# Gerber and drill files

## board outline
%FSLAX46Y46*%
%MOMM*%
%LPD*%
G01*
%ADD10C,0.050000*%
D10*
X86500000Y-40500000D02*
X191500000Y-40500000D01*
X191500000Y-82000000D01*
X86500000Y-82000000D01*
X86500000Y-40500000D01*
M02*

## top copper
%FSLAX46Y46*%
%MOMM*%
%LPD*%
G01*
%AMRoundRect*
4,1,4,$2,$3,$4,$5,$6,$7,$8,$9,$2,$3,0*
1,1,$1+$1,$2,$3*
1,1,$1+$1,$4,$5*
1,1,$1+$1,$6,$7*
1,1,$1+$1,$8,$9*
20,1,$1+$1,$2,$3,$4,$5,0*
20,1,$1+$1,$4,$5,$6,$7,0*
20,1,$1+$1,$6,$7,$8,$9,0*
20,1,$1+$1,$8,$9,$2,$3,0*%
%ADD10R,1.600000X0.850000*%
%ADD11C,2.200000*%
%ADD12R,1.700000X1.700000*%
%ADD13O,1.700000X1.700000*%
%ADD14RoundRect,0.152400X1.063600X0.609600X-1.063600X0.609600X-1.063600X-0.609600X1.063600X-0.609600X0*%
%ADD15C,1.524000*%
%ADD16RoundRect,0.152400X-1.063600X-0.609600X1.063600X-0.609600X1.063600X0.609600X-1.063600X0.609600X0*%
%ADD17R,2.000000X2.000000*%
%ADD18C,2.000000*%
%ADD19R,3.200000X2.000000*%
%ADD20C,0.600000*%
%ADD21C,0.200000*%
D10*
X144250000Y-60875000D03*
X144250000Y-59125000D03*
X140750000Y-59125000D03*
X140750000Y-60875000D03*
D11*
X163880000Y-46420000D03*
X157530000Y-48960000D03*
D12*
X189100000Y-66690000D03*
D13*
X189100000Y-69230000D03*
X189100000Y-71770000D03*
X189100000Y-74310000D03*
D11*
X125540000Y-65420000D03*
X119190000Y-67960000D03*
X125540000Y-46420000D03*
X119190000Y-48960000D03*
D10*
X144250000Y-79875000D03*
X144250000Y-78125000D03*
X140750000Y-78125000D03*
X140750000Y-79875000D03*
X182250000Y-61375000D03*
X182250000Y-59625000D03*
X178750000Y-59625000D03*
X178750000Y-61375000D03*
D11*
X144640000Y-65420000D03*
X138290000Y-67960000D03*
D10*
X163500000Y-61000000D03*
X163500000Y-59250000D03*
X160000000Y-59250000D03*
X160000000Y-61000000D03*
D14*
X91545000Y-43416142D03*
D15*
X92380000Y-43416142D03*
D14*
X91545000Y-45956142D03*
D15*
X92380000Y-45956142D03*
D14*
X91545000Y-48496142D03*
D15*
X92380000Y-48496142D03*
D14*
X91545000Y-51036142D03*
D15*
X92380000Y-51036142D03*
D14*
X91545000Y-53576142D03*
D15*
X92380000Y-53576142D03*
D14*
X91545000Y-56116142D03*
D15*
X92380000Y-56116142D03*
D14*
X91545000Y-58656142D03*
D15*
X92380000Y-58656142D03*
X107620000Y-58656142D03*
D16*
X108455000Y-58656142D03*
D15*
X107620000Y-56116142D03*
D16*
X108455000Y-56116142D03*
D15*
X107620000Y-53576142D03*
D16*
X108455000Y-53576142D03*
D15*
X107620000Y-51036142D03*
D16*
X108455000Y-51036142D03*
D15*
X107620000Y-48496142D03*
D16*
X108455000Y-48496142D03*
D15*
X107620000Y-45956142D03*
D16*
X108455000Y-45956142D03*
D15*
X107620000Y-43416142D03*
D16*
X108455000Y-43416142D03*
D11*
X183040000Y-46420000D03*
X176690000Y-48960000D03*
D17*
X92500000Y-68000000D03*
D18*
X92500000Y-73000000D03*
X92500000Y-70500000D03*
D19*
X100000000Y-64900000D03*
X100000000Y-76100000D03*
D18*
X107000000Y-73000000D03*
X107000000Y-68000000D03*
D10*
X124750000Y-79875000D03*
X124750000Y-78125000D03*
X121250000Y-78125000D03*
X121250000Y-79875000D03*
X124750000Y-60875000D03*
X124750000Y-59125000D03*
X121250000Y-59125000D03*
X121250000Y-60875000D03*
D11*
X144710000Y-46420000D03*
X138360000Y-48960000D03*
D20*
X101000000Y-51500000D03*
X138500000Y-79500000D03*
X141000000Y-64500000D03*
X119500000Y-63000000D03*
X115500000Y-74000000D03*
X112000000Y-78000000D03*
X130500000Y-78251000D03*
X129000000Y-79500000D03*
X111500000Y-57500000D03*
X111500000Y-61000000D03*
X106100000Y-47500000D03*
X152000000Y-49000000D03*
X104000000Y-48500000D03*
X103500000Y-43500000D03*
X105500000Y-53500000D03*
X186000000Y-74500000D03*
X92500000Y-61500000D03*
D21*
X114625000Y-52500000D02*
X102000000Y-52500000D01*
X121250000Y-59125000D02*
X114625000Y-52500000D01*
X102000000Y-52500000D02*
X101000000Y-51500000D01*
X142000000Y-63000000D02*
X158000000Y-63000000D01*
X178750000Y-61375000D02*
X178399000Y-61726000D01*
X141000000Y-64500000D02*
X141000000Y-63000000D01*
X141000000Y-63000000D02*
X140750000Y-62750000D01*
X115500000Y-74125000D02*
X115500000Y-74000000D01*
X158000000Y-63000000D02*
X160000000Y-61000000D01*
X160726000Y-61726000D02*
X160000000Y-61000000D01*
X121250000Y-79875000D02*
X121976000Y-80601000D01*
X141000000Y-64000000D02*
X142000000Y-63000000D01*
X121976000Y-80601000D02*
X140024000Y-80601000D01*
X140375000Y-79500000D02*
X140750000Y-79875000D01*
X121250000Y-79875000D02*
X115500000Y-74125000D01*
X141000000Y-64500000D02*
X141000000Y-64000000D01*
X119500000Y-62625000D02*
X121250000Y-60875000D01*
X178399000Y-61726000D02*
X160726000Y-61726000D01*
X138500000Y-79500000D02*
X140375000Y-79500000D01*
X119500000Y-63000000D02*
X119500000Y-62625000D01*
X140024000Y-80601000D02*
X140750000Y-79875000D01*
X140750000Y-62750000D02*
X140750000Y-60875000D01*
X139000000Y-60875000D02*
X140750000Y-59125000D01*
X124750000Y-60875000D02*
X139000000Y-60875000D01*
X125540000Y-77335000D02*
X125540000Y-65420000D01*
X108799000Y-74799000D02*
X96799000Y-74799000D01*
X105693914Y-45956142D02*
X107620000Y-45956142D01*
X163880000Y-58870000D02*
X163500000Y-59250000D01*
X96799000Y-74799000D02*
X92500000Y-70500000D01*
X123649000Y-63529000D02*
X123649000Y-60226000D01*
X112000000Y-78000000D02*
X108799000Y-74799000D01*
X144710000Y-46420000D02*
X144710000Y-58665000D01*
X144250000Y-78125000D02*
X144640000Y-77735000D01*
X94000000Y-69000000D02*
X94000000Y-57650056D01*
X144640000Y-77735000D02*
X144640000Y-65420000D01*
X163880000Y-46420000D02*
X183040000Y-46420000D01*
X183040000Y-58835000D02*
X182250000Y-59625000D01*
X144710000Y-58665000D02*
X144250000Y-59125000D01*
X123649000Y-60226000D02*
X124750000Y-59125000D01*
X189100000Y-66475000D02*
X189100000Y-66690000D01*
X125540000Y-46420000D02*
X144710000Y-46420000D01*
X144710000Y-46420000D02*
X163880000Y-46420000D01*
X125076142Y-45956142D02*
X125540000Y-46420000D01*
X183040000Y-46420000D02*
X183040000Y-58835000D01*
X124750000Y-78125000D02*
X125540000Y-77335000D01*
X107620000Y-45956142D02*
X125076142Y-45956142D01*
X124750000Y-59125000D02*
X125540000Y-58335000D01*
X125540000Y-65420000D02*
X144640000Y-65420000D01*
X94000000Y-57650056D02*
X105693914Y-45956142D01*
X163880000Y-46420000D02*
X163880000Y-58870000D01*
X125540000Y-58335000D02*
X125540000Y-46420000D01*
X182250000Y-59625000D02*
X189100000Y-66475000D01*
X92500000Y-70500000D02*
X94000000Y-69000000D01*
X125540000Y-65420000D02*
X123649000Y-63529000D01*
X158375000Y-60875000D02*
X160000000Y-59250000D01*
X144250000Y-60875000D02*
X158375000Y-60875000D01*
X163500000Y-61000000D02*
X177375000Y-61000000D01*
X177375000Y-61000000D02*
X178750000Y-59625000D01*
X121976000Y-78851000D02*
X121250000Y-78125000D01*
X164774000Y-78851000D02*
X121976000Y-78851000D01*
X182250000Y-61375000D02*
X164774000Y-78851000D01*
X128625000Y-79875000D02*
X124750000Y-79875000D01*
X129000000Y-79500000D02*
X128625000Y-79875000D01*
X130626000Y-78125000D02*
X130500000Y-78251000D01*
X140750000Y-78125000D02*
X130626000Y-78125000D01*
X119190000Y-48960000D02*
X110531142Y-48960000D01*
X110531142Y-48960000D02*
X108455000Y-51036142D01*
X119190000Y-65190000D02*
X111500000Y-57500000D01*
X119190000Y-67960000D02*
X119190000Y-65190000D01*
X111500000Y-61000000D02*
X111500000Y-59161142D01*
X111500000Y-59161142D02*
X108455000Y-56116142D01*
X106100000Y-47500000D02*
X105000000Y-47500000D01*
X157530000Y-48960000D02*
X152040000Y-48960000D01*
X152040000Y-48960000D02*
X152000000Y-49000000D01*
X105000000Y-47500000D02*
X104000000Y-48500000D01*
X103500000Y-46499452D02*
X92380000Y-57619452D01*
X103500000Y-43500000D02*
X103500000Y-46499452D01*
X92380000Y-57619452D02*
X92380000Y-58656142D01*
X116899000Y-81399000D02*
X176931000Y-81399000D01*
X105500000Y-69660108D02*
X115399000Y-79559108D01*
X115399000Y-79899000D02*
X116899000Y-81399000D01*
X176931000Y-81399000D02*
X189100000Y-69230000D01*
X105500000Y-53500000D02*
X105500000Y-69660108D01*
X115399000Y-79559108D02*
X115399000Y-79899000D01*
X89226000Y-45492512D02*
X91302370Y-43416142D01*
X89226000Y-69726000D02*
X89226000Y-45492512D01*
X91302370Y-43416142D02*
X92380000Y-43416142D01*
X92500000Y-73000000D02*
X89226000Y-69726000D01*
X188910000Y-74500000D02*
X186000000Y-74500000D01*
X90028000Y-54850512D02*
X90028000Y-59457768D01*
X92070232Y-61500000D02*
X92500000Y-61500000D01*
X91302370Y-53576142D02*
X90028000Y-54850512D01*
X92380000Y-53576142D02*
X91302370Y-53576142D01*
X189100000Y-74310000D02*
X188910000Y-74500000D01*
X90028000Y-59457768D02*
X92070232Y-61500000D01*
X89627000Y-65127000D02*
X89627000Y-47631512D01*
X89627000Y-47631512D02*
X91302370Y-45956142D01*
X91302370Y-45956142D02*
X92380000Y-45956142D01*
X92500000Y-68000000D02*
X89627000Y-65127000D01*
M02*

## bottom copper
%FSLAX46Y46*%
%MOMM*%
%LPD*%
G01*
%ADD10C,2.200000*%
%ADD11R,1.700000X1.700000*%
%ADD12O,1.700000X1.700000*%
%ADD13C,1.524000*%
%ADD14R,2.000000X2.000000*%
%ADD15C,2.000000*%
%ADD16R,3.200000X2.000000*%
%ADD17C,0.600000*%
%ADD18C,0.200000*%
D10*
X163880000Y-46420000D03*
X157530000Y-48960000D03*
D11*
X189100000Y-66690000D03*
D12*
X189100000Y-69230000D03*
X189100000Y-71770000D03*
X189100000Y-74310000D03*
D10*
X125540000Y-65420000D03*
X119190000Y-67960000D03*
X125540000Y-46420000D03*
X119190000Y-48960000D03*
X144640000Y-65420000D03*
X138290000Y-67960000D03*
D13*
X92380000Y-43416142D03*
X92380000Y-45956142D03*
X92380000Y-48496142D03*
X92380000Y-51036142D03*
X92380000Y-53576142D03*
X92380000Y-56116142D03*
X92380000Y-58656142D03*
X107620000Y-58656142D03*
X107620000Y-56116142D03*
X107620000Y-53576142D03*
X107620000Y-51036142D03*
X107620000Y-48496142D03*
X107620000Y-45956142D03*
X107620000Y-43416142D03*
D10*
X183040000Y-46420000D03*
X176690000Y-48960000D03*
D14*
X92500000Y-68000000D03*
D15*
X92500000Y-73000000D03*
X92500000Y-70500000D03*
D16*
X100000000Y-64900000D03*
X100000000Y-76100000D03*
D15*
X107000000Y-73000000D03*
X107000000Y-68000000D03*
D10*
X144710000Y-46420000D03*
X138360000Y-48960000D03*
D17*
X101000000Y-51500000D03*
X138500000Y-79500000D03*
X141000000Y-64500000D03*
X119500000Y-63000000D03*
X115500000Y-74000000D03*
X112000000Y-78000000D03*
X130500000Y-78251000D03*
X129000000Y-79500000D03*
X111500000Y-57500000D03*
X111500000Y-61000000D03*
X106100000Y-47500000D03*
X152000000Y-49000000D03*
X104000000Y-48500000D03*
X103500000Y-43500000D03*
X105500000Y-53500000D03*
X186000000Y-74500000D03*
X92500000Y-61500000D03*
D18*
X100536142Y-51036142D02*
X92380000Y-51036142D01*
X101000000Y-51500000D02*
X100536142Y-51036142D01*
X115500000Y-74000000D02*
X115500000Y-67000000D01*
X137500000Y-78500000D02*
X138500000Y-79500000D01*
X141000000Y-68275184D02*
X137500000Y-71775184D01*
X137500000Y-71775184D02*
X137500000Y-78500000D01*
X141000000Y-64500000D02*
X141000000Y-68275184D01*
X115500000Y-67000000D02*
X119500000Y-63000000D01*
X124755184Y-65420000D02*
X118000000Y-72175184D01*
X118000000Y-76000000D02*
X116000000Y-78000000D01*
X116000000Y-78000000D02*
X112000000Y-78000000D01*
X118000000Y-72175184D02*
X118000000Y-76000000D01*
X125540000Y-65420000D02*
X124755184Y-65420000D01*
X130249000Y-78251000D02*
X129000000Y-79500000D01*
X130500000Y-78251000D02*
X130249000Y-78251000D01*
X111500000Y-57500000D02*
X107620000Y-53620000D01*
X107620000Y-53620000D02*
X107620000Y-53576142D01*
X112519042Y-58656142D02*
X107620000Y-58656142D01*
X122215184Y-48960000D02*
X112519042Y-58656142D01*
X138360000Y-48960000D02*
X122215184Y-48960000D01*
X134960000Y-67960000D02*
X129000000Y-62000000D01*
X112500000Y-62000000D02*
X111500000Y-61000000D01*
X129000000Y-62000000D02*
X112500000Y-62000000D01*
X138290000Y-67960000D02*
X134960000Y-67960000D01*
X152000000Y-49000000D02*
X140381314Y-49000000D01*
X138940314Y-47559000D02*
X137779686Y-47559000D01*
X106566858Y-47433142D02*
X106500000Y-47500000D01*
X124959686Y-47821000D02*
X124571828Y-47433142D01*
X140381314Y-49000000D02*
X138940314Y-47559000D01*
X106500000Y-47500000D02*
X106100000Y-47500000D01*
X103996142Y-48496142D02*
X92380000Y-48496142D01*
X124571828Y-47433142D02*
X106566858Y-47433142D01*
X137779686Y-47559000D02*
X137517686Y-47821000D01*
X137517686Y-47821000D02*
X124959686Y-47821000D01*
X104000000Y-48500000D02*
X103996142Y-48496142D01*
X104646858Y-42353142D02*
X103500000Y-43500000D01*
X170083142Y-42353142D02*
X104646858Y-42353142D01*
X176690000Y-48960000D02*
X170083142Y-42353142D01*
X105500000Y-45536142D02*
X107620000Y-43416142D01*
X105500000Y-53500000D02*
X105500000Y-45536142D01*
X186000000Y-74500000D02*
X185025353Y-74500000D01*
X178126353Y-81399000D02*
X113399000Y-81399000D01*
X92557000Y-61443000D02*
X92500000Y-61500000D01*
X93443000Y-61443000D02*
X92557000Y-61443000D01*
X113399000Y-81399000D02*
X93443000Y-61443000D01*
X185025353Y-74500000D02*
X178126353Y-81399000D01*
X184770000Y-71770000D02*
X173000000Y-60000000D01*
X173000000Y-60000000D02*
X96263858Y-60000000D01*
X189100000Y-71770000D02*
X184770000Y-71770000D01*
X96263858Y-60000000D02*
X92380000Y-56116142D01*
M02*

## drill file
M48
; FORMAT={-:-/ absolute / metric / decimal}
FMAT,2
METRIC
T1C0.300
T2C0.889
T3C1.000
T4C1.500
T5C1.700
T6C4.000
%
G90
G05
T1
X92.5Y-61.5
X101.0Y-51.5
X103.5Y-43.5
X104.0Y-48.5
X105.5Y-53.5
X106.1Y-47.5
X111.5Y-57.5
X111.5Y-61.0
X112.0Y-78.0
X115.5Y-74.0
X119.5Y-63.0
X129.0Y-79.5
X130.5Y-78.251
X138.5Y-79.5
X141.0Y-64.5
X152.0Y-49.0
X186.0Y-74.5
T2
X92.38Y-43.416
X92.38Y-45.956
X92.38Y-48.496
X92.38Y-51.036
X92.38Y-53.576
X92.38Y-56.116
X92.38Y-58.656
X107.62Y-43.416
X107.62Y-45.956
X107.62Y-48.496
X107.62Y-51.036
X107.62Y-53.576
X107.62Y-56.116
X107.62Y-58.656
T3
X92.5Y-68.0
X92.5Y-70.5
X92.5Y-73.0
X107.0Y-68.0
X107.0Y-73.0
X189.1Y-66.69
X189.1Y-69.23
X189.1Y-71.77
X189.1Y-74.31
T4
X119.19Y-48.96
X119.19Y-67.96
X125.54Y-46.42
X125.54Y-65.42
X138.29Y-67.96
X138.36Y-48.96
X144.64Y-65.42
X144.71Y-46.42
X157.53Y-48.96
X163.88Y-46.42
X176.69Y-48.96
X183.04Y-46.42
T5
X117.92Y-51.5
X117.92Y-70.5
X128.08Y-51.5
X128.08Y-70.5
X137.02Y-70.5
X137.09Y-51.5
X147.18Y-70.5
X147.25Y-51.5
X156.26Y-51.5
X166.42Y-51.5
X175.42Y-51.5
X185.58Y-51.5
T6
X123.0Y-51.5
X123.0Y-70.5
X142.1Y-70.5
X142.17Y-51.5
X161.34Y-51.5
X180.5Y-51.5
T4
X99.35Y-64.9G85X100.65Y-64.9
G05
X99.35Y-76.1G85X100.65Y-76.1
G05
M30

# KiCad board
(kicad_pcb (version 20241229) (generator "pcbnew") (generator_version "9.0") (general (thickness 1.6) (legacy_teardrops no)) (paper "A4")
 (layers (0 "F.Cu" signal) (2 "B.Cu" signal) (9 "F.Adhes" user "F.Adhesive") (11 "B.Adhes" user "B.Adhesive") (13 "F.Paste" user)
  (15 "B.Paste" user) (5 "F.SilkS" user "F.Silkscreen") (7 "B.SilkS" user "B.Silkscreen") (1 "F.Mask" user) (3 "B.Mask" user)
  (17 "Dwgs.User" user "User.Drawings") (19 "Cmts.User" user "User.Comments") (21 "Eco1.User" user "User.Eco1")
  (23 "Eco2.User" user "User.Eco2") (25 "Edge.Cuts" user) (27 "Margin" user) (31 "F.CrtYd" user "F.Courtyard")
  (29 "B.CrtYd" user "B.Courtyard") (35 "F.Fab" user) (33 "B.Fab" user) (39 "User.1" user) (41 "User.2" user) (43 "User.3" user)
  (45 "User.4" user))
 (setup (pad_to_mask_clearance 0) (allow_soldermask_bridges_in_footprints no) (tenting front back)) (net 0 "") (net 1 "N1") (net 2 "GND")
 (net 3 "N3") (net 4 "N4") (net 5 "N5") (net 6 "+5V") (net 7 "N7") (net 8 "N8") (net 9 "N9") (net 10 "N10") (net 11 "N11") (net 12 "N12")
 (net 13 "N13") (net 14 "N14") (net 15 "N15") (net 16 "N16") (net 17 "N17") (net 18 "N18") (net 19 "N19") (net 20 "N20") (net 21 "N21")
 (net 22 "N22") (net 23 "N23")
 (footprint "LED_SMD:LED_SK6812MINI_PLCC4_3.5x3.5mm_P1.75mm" (layer "F.Cu") (at 142.5 60 180)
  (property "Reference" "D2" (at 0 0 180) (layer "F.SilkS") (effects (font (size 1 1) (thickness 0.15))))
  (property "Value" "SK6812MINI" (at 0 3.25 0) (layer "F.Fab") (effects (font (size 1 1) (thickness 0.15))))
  (pad "1" smd rect (at -1.75 -0.875 180) (size 1.6 0.85) (layers "F.Cu" "F.Mask" "F.Paste") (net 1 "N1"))
  (pad "2" smd rect (at -1.75 0.875 180) (size 1.6 0.85) (layers "F.Cu" "F.Mask" "F.Paste") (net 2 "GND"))
  (pad "3" smd rect (at 1.75 0.875 180) (size 1.6 0.85) (layers "F.Cu" "F.Mask" "F.Paste") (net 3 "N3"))
  (pad "4" smd rect (at 1.75 -0.875 180) (size 1.6 0.85) (layers "F.Cu" "F.Mask" "F.Paste") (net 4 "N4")))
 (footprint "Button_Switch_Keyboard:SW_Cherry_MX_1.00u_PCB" (layer "F.Cu") (at 163.88 46.42)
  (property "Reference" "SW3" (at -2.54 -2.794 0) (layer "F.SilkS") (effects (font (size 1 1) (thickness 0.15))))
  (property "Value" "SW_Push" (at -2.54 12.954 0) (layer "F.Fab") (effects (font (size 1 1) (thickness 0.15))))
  (pad "" np_thru_hole circle (at -7.62 5.08) (size 1.7 1.7) (drill 1.7) (layers "*.Cu" "*.Mask"))
  (pad "" np_thru_hole circle (at -2.54 5.08) (size 4 4) (drill 4) (layers "*.Cu" "*.Mask"))
  (pad "" np_thru_hole circle (at 2.54 5.08) (size 1.7 1.7) (drill 1.7) (layers "*.Cu" "*.Mask"))
  (pad "1" thru_hole circle (at 0 0) (size 2.2 2.2) (drill 1.5) (layers "*.Cu" "*.Mask") (remove_unused_layers no) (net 2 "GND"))
  (pad "2" thru_hole circle (at -6.35 2.54) (size 2.2 2.2) (drill 1.5) (layers "*.Cu" "*.Mask") (remove_unused_layers no) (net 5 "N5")))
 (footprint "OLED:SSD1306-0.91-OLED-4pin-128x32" (layer "F.Cu") (at 152.6 64.5)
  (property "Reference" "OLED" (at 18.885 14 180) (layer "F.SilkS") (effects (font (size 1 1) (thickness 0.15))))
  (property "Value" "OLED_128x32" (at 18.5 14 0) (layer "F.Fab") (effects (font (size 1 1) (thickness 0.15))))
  (pad "1" thru_hole rect (at 36.5 2.19) (size 1.7 1.7) (drill 1) (layers "*.Cu" "*.Mask") (remove_unused_layers no) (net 2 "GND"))
  (pad "2" thru_hole oval (at 36.5 4.73) (size 1.7 1.7) (drill 1) (layers "*.Cu" "*.Mask") (remove_unused_layers no) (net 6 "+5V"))
  (pad "3" thru_hole oval (at 36.5 7.27) (size 1.7 1.7) (drill 1) (layers "*.Cu" "*.Mask") (remove_unused_layers no) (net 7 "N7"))
  (pad "4" thru_hole oval (at 36.5 9.81) (size 1.7 1.7) (drill 1) (layers "*.Cu" "*.Mask") (remove_unused_layers no) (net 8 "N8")))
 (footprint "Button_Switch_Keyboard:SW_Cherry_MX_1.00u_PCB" (layer "F.Cu") (at 125.54 65.42)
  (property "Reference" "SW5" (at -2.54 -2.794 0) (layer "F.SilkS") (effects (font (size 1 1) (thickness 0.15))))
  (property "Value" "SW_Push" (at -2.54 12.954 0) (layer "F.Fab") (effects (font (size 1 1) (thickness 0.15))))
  (pad "" np_thru_hole circle (at -7.62 5.08) (size 1.7 1.7) (drill 1.7) (layers "*.Cu" "*.Mask"))
  (pad "" np_thru_hole circle (at -2.54 5.08) (size 4 4) (drill 4) (layers "*.Cu" "*.Mask"))
  (pad "" np_thru_hole circle (at 2.54 5.08) (size 1.7 1.7) (drill 1.7) (layers "*.Cu" "*.Mask"))
  (pad "1" thru_hole circle (at 0 0) (size 2.2 2.2) (drill 1.5) (layers "*.Cu" "*.Mask") (remove_unused_layers no) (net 2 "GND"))
  (pad "2" thru_hole circle (at -6.35 2.54) (size 2.2 2.2) (drill 1.5) (layers "*.Cu" "*.Mask") (remove_unused_layers no) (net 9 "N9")))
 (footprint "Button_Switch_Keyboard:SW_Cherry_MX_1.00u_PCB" (layer "F.Cu") (at 125.54 46.42)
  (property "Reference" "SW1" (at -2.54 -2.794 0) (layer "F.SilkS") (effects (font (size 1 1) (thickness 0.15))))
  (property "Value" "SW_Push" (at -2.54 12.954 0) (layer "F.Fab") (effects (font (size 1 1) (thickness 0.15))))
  (pad "" np_thru_hole circle (at -7.62 5.08) (size 1.7 1.7) (drill 1.7) (layers "*.Cu" "*.Mask"))
  (pad "" np_thru_hole circle (at -2.54 5.08) (size 4 4) (drill 4) (layers "*.Cu" "*.Mask"))
  (pad "" np_thru_hole circle (at 2.54 5.08) (size 1.7 1.7) (drill 1.7) (layers "*.Cu" "*.Mask"))
  (pad "1" thru_hole circle (at 0 0) (size 2.2 2.2) (drill 1.5) (layers "*.Cu" "*.Mask") (remove_unused_layers no) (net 2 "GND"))
  (pad "2" thru_hole circle (at -6.35 2.54) (size 2.2 2.2) (drill 1.5) (layers "*.Cu" "*.Mask") (remove_unused_layers no) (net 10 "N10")))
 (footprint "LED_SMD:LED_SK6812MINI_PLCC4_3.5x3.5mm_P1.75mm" (layer "F.Cu") (at 142.5 79 180)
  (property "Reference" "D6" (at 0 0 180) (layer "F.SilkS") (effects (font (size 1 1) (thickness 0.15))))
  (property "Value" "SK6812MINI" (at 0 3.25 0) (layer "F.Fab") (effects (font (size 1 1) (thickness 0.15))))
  (pad "1" smd rect (at -1.75 -0.875 180) (size 1.6 0.85) (layers "F.Cu" "F.Mask" "F.Paste") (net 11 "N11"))
  (pad "2" smd rect (at -1.75 0.875 180) (size 1.6 0.85) (layers "F.Cu" "F.Mask" "F.Paste") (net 2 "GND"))
  (pad "3" smd rect (at 1.75 0.875 180) (size 1.6 0.85) (layers "F.Cu" "F.Mask" "F.Paste") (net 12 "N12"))
  (pad "4" smd rect (at 1.75 -0.875 180) (size 1.6 0.85) (layers "F.Cu" "F.Mask" "F.Paste") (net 4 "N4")))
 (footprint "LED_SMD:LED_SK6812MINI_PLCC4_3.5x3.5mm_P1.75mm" (layer "F.Cu") (at 180.5 60.5 180)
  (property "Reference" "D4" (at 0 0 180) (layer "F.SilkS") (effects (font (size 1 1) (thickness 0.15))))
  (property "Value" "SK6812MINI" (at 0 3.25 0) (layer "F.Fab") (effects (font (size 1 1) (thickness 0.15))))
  (pad "1" smd rect (at -1.75 -0.875 180) (size 1.6 0.85) (layers "F.Cu" "F.Mask" "F.Paste") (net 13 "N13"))
  (pad "2" smd rect (at -1.75 0.875 180) (size 1.6 0.85) (layers "F.Cu" "F.Mask" "F.Paste") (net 2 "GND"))
  (pad "3" smd rect (at 1.75 0.875 180) (size 1.6 0.85) (layers "F.Cu" "F.Mask" "F.Paste") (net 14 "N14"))
  (pad "4" smd rect (at 1.75 -0.875 180) (size 1.6 0.85) (layers "F.Cu" "F.Mask" "F.Paste") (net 4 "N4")))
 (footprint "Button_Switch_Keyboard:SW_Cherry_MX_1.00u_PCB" (layer "F.Cu") (at 144.64 65.42)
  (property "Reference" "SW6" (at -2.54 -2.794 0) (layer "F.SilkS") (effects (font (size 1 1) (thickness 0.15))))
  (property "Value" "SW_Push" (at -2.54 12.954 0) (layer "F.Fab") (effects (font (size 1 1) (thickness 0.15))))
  (pad "" np_thru_hole circle (at -7.62 5.08) (size 1.7 1.7) (drill 1.7) (layers "*.Cu" "*.Mask"))
  (pad "" np_thru_hole circle (at -2.54 5.08) (size 4 4) (drill 4) (layers "*.Cu" "*.Mask"))
  (pad "" np_thru_hole circle (at 2.54 5.08) (size 1.7 1.7) (drill 1.7) (layers "*.Cu" "*.Mask"))
  (pad "1" thru_hole circle (at 0 0) (size 2.2 2.2) (drill 1.5) (layers "*.Cu" "*.Mask") (remove_unused_layers no) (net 2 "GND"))
  (pad "2" thru_hole circle (at -6.35 2.54) (size 2.2 2.2) (drill 1.5) (layers "*.Cu" "*.Mask") (remove_unused_layers no) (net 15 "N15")))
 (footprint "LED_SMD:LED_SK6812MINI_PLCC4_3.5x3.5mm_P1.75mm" (layer "F.Cu") (at 161.75 60.125 180)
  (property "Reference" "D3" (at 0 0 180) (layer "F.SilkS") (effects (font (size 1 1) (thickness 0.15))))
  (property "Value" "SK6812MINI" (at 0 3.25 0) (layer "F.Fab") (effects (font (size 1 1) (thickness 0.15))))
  (pad "1" smd rect (at -1.75 -0.875 180) (size 1.6 0.85) (layers "F.Cu" "F.Mask" "F.Paste") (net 14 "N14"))
  (pad "2" smd rect (at -1.75 0.875 180) (size 1.6 0.85) (layers "F.Cu" "F.Mask" "F.Paste") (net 2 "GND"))
  (pad "3" smd rect (at 1.75 0.875 180) (size 1.6 0.85) (layers "F.Cu" "F.Mask" "F.Paste") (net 1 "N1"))
  (pad "4" smd rect (at 1.75 -0.875 180) (size 1.6 0.85) (layers "F.Cu" "F.Mask" "F.Paste") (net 4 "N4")))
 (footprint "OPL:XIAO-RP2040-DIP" (layer "F.Cu") (at 100 51.036142)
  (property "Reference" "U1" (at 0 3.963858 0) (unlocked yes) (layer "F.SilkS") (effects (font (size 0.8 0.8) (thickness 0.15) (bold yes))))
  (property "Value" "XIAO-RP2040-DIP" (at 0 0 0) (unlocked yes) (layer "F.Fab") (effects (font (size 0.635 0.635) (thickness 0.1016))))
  (pad "1" smd roundrect (at -8.455 -7.62 180) (size 2.432 1.524) (layers "F.Cu" "F.Mask") (roundrect_rratio 0.1) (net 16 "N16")
   (thermal_bridge_angle 45))
  (pad "1" thru_hole circle (at -7.62 -7.62 180) (size 1.524 1.524) (drill 0.889) (layers "*.Cu" "*.Mask") (remove_unused_layers no)
   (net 16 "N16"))
  (pad "2" smd roundrect (at -8.455 -5.08 180) (size 2.432 1.524) (layers "F.Cu" "F.Mask") (roundrect_rratio 0.1) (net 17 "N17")
   (thermal_bridge_angle 45))
  (pad "2" thru_hole circle (at -7.62 -5.08 180) (size 1.524 1.524) (drill 0.889) (layers "*.Cu" "*.Mask") (remove_unused_layers no)
   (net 17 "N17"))
  (pad "3" smd roundrect (at -8.455 -2.54 180) (size 2.432 1.524) (layers "F.Cu" "F.Mask") (roundrect_rratio 0.1) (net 5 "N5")
   (thermal_bridge_angle 45))
  (pad "3" thru_hole circle (at -7.62 -2.54 180) (size 1.524 1.524) (drill 0.889) (layers "*.Cu" "*.Mask") (remove_unused_layers no)
   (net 5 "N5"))
  (pad "4" smd roundrect (at -8.455 0 180) (size 2.432 1.524) (layers "F.Cu" "F.Mask") (roundrect_rratio 0.1) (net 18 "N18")
   (thermal_bridge_angle 45))
  (pad "4" thru_hole circle (at -7.62 0 180) (size 1.524 1.524) (drill 0.889) (layers "*.Cu" "*.Mask") (remove_unused_layers no)
   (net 18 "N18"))
  (pad "5" smd roundrect (at -8.455 2.54 180) (size 2.432 1.524) (layers "F.Cu" "F.Mask") (roundrect_rratio 0.1) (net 8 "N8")
   (thermal_bridge_angle 45))
  (pad "5" thru_hole circle (at -7.62 2.54 180) (size 1.524 1.524) (drill 0.889) (layers "*.Cu" "*.Mask") (remove_unused_layers no)
   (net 8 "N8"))
  (pad "6" smd roundrect (at -8.455 5.08 180) (size 2.432 1.524) (layers "F.Cu" "F.Mask") (roundrect_rratio 0.1) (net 7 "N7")
   (thermal_bridge_angle 45))
  (pad "6" thru_hole circle (at -7.62 5.08 180) (size 1.524 1.524) (drill 0.889) (layers "*.Cu" "*.Mask") (remove_unused_layers no)
   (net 7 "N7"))
  (pad "7" smd roundrect (at -8.455 7.62 180) (size 2.432 1.524) (layers "F.Cu" "F.Mask") (roundrect_rratio 0.1) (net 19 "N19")
   (thermal_bridge_angle 45))
  (pad "7" thru_hole circle (at -7.62 7.62 180) (size 1.524 1.524) (drill 0.889) (layers "*.Cu" "*.Mask") (remove_unused_layers no)
   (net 19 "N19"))
  (pad "8" thru_hole circle (at 7.62 7.62) (size 1.524 1.524) (drill 0.889) (layers "*.Cu" "*.Mask") (remove_unused_layers no)
   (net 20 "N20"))
  (pad "8" smd roundrect (at 8.455 7.62) (size 2.432 1.524) (layers "F.Cu" "F.Mask") (roundrect_rratio 0.1) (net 20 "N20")
   (thermal_bridge_angle 45))
  (pad "9" thru_hole circle (at 7.62 5.08) (size 1.524 1.524) (drill 0.889) (layers "*.Cu" "*.Mask") (remove_unused_layers no)
   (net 15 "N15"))
  (pad "9" smd roundrect (at 8.455 5.08) (size 2.432 1.524) (layers "F.Cu" "F.Mask") (roundrect_rratio 0.1) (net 15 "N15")
   (thermal_bridge_angle 45))
  (pad "10" thru_hole circle (at 7.62 2.54) (size 1.524 1.524) (drill 0.889) (layers "*.Cu" "*.Mask") (remove_unused_layers no) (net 9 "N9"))
  (pad "10" smd roundrect (at 8.455 2.54) (size 2.432 1.524) (layers "F.Cu" "F.Mask") (roundrect_rratio 0.1) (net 9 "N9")
   (thermal_bridge_angle 45))
  (pad "11" thru_hole circle (at 7.62 0) (size 1.524 1.524) (drill 0.889) (layers "*.Cu" "*.Mask") (remove_unused_layers no) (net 10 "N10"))
  (pad "11" smd roundrect (at 8.455 0) (size 2.432 1.524) (layers "F.Cu" "F.Mask") (roundrect_rratio 0.1) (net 10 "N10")
   (thermal_bridge_angle 45))
  (pad "12" thru_hole circle (at 7.62 -2.54) (size 1.524 1.524) (drill 0.889) (layers "*.Cu" "*.Mask") (remove_unused_layers no)
   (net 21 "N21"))
  (pad "12" smd roundrect (at 8.455 -2.54) (size 2.432 1.524) (layers "F.Cu" "F.Mask") (roundrect_rratio 0.1) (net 21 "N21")
   (thermal_bridge_angle 45))
  (pad "13" thru_hole circle (at 7.62 -5.08) (size 1.524 1.524) (drill 0.889) (layers "*.Cu" "*.Mask") (remove_unused_layers no)
   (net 2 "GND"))
  (pad "13" smd roundrect (at 8.455 -5.08) (size 2.432 1.524) (layers "F.Cu" "F.Mask") (roundrect_rratio 0.1) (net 2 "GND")
   (thermal_bridge_angle 45))
  (pad "14" thru_hole circle (at 7.62 -7.62) (size 1.524 1.524) (drill 0.889) (layers "*.Cu" "*.Mask") (remove_unused_layers no)
   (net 6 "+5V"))
  (pad "14" smd roundrect (at 8.455 -7.62) (size 2.432 1.524) (layers "F.Cu" "F.Mask") (roundrect_rratio 0.1) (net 6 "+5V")
   (thermal_bridge_angle 45)))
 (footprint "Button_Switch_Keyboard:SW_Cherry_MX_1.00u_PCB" (layer "F.Cu") (at 183.04 46.42)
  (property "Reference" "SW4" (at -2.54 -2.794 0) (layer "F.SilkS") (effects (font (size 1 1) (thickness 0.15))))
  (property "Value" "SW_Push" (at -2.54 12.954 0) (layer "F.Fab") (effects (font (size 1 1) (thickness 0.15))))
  (pad "" np_thru_hole circle (at -7.62 5.08) (size 1.7 1.7) (drill 1.7) (layers "*.Cu" "*.Mask"))
  (pad "" np_thru_hole circle (at -2.54 5.08) (size 4 4) (drill 4) (layers "*.Cu" "*.Mask"))
  (pad "" np_thru_hole circle (at 2.54 5.08) (size 1.7 1.7) (drill 1.7) (layers "*.Cu" "*.Mask"))
  (pad "1" thru_hole circle (at 0 0) (size 2.2 2.2) (drill 1.5) (layers "*.Cu" "*.Mask") (remove_unused_layers no) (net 2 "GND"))
  (pad "2" thru_hole circle (at -6.35 2.54) (size 2.2 2.2) (drill 1.5) (layers "*.Cu" "*.Mask") (remove_unused_layers no) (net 19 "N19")))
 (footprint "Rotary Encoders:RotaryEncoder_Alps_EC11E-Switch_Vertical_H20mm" (layer "F.Cu") (at 92.5 68)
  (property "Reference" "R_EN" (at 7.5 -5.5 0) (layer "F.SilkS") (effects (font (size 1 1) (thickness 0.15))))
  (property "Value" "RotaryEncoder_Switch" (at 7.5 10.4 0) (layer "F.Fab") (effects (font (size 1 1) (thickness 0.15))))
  (pad "A" thru_hole rect (at 0 0) (size 2 2) (drill 1) (layers "*.Cu" "*.Mask") (remove_unused_layers no) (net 17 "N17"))
  (pad "B" thru_hole circle (at 0 5) (size 2 2) (drill 1) (layers "*.Cu" "*.Mask") (remove_unused_layers no) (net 16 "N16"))
  (pad "C" thru_hole circle (at 0 2.5) (size 2 2) (drill 1) (layers "*.Cu" "*.Mask") (remove_unused_layers no) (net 2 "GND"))
  (pad "MP" thru_hole rect (at 7.5 -3.1) (size 3.2 2) (drill oval 2.8 1.5) (layers "*.Cu" "*.Mask") (remove_unused_layers no))
  (pad "MP" thru_hole rect (at 7.5 8.1) (size 3.2 2) (drill oval 2.8 1.5) (layers "*.Cu" "*.Mask") (remove_unused_layers no))
  (pad "S1" thru_hole circle (at 14.5 5) (size 2 2) (drill 1) (layers "*.Cu" "*.Mask") (remove_unused_layers no) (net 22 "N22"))
  (pad "S2" thru_hole circle (at 14.5 0) (size 2 2) (drill 1) (layers "*.Cu" "*.Mask") (remove_unused_layers no) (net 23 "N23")))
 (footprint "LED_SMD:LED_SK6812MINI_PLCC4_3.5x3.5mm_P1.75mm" (layer "F.Cu") (at 123 79 180)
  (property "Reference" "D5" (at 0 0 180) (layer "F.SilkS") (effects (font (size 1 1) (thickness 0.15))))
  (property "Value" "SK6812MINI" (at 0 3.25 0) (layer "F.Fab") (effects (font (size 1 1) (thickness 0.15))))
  (pad "1" smd rect (at -1.75 -0.875 180) (size 1.6 0.85) (layers "F.Cu" "F.Mask" "F.Paste") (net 12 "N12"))
  (pad "2" smd rect (at -1.75 0.875 180) (size 1.6 0.85) (layers "F.Cu" "F.Mask" "F.Paste") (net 2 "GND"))
  (pad "3" smd rect (at 1.75 0.875 180) (size 1.6 0.85) (layers "F.Cu" "F.Mask" "F.Paste") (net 13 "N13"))
  (pad "4" smd rect (at 1.75 -0.875 180) (size 1.6 0.85) (layers "F.Cu" "F.Mask" "F.Paste") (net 4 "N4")))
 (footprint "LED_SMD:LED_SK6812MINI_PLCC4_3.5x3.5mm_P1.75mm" (layer "F.Cu") (at 123 60 180)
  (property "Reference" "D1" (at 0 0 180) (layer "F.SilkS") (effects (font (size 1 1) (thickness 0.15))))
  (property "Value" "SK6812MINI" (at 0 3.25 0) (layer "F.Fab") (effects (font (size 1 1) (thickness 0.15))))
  (pad "1" smd rect (at -1.75 -0.875 180) (size 1.6 0.85) (layers "F.Cu" "F.Mask" "F.Paste") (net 3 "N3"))
  (pad "2" smd rect (at -1.75 0.875 180) (size 1.6 0.85) (layers "F.Cu" "F.Mask" "F.Paste") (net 2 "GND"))
  (pad "3" smd rect (at 1.75 0.875 180) (size 1.6 0.85) (layers "F.Cu" "F.Mask" "F.Paste") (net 18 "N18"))
  (pad "4" smd rect (at 1.75 -0.875 180) (size 1.6 0.85) (layers "F.Cu" "F.Mask" "F.Paste") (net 4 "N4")))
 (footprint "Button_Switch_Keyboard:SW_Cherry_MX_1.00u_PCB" (layer "F.Cu") (at 144.71 46.42)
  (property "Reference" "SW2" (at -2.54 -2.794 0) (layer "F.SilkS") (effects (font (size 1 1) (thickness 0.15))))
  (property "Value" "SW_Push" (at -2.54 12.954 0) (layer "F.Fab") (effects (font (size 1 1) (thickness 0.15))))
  (pad "" np_thru_hole circle (at -7.62 5.08) (size 1.7 1.7) (drill 1.7) (layers "*.Cu" "*.Mask"))
  (pad "" np_thru_hole circle (at -2.54 5.08) (size 4 4) (drill 4) (layers "*.Cu" "*.Mask"))
  (pad "" np_thru_hole circle (at 2.54 5.08) (size 1.7 1.7) (drill 1.7) (layers "*.Cu" "*.Mask"))
  (pad "1" thru_hole circle (at 0 0) (size 2.2 2.2) (drill 1.5) (layers "*.Cu" "*.Mask") (remove_unused_layers no) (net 2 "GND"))
  (pad "2" thru_hole circle (at -6.35 2.54) (size 2.2 2.2) (drill 1.5) (layers "*.Cu" "*.Mask") (remove_unused_layers no) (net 20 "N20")))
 (gr_rect (start 86.5 40.5) (end 191.5 82) (stroke (width 0.05) (type default)) (fill no) (layer "Edge.Cuts"))
 (segment (start 114.625 52.5) (end 102 52.5) (width 0.2) (layer "F.Cu") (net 18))
 (segment (start 121.25 59.125) (end 114.625 52.5) (width 0.2) (layer "F.Cu") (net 18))
 (segment (start 102 52.5) (end 101 51.5) (width 0.2) (layer "F.Cu") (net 18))
 (via (at 101 51.5) (size 0.6) (drill 0.3) (layers "F.Cu" "B.Cu") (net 18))
 (segment (start 100.536142 51.036142) (end 92.38 51.036142) (width 0.2) (layer "B.Cu") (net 18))
 (segment (start 101 51.5) (end 100.536142 51.036142) (width 0.2) (layer "B.Cu") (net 18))
 (segment (start 142 63) (end 158 63) (width 0.2) (layer "F.Cu") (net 4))
 (segment (start 178.75 61.375) (end 178.399 61.726) (width 0.2) (layer "F.Cu") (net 4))
 (segment (start 141 64.5) (end 141 63) (width 0.2) (layer "F.Cu") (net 4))
 (segment (start 141 63) (end 140.75 62.75) (width 0.2) (layer "F.Cu") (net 4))
 (segment (start 115.5 74.125) (end 115.5 74) (width 0.2) (layer "F.Cu") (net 4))
 (segment (start 158 63) (end 160 61) (width 0.2) (layer "F.Cu") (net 4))
 (segment (start 160.726 61.726) (end 160 61) (width 0.2) (layer "F.Cu") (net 4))
 (segment (start 121.25 79.875) (end 121.976 80.601) (width 0.2) (layer "F.Cu") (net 4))
 (segment (start 141 64) (end 142 63) (width 0.2) (layer "F.Cu") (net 4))
 (segment (start 121.976 80.601) (end 140.024 80.601) (width 0.2) (layer "F.Cu") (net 4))
 (segment (start 140.375 79.5) (end 140.75 79.875) (width 0.2) (layer "F.Cu") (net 4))
 (segment (start 121.25 79.875) (end 115.5 74.125) (width 0.2) (layer "F.Cu") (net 4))
 (segment (start 141 64.5) (end 141 64) (width 0.2) (layer "F.Cu") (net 4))
 (segment (start 119.5 62.625) (end 121.25 60.875) (width 0.2) (layer "F.Cu") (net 4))
 (segment (start 178.399 61.726) (end 160.726 61.726) (width 0.2) (layer "F.Cu") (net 4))
 (segment (start 138.5 79.5) (end 140.375 79.5) (width 0.2) (layer "F.Cu") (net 4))
 (segment (start 119.5 63) (end 119.5 62.625) (width 0.2) (layer "F.Cu") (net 4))
 (segment (start 140.024 80.601) (end 140.75 79.875) (width 0.2) (layer "F.Cu") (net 4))
 (segment (start 140.75 62.75) (end 140.75 60.875) (width 0.2) (layer "F.Cu") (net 4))
 (via (at 138.5 79.5) (size 0.6) (drill 0.3) (layers "F.Cu" "B.Cu") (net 4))
 (via (at 141 64.5) (size 0.6) (drill 0.3) (layers "F.Cu" "B.Cu") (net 4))
 (via (at 119.5 63) (size 0.6) (drill 0.3) (layers "F.Cu" "B.Cu") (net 4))
 (via (at 115.5 74) (size 0.6) (drill 0.3) (layers "F.Cu" "B.Cu") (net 4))
 (segment (start 115.5 74) (end 115.5 67) (width 0.2) (layer "B.Cu") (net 4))
 (segment (start 137.5 78.5) (end 138.5 79.5) (width 0.2) (layer "B.Cu") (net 4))
 (segment (start 141 68.275184) (end 137.5 71.775184) (width 0.2) (layer "B.Cu") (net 4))
 (segment (start 137.5 71.775184) (end 137.5 78.5) (width 0.2) (layer "B.Cu") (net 4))
 (segment (start 141 64.5) (end 141 68.275184) (width 0.2) (layer "B.Cu") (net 4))
 (segment (start 115.5 67) (end 119.5 63) (width 0.2) (layer "B.Cu") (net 4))
 (segment (start 139 60.875) (end 140.75 59.125) (width 0.2) (layer "F.Cu") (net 3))
 (segment (start 124.75 60.875) (end 139 60.875) (width 0.2) (layer "F.Cu") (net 3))
 (segment (start 125.54 77.335) (end 125.54 65.42) (width 0.2) (layer "F.Cu") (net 2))
 (segment (start 108.799 74.799) (end 96.799 74.799) (width 0.2) (layer "F.Cu") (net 2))
 (segment (start 105.693914 45.956142) (end 107.62 45.956142) (width 0.2) (layer "F.Cu") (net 2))
 (segment (start 163.88 58.87) (end 163.5 59.25) (width 0.2) (layer "F.Cu") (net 2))
 (segment (start 96.799 74.799) (end 92.5 70.5) (width 0.2) (layer "F.Cu") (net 2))
 (segment (start 123.649 63.529) (end 123.649 60.226) (width 0.2) (layer "F.Cu") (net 2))
 (segment (start 112 78) (end 108.799 74.799) (width 0.2) (layer "F.Cu") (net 2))
 (segment (start 144.71 46.42) (end 144.71 58.665) (width 0.2) (layer "F.Cu") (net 2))
 (segment (start 144.25 78.125) (end 144.64 77.735) (width 0.2) (layer "F.Cu") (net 2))
 (segment (start 94 69) (end 94 57.650056) (width 0.2) (layer "F.Cu") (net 2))
 (segment (start 144.64 77.735) (end 144.64 65.42) (width 0.2) (layer "F.Cu") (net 2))
 (segment (start 163.88 46.42) (end 183.04 46.42) (width 0.2) (layer "F.Cu") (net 2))
 (segment (start 183.04 58.835) (end 182.25 59.625) (width 0.2) (layer "F.Cu") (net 2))
 (segment (start 144.71 58.665) (end 144.25 59.125) (width 0.2) (layer "F.Cu") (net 2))
 (segment (start 123.649 60.226) (end 124.75 59.125) (width 0.2) (layer "F.Cu") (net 2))
 (segment (start 189.1 66.475) (end 189.1 66.69) (width 0.2) (layer "F.Cu") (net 2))
 (segment (start 125.54 46.42) (end 144.71 46.42) (width 0.2) (layer "F.Cu") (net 2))
 (segment (start 144.71 46.42) (end 163.88 46.42) (width 0.2) (layer "F.Cu") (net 2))
 (segment (start 125.076142 45.956142) (end 125.54 46.42) (width 0.2) (layer "F.Cu") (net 2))
 (segment (start 183.04 46.42) (end 183.04 58.835) (width 0.2) (layer "F.Cu") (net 2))
 (segment (start 124.75 78.125) (end 125.54 77.335) (width 0.2) (layer "F.Cu") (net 2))
 (segment (start 107.62 45.956142) (end 125.076142 45.956142) (width 0.2) (layer "F.Cu") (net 2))
 (segment (start 124.75 59.125) (end 125.54 58.335) (width 0.2) (layer "F.Cu") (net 2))
 (segment (start 125.54 65.42) (end 144.64 65.42) (width 0.2) (layer "F.Cu") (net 2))
 (segment (start 94 57.650056) (end 105.693914 45.956142) (width 0.2) (layer "F.Cu") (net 2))
 (segment (start 163.88 46.42) (end 163.88 58.87) (width 0.2) (layer "F.Cu") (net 2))
 (segment (start 125.54 58.335) (end 125.54 46.42) (width 0.2) (layer "F.Cu") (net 2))
 (segment (start 182.25 59.625) (end 189.1 66.475) (width 0.2) (layer "F.Cu") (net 2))
 (segment (start 92.5 70.5) (end 94 69) (width 0.2) (layer "F.Cu") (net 2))
 (segment (start 125.54 65.42) (end 123.649 63.529) (width 0.2) (layer "F.Cu") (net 2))
 (via (at 112 78) (size 0.6) (drill 0.3) (layers "F.Cu" "B.Cu") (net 2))
 (segment (start 124.755184 65.42) (end 118 72.175184) (width 0.2) (layer "B.Cu") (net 2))
 (segment (start 118 76) (end 116 78) (width 0.2) (layer "B.Cu") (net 2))
 (segment (start 116 78) (end 112 78) (width 0.2) (layer "B.Cu") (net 2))
 (segment (start 118 72.175184) (end 118 76) (width 0.2) (layer "B.Cu") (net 2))
 (segment (start 125.54 65.42) (end 124.755184 65.42) (width 0.2) (layer "B.Cu") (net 2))
 (segment (start 158.375 60.875) (end 160 59.25) (width 0.2) (layer "F.Cu") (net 1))
 (segment (start 144.25 60.875) (end 158.375 60.875) (width 0.2) (layer "F.Cu") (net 1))
 (segment (start 163.5 61) (end 177.375 61) (width 0.2) (layer "F.Cu") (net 14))
 (segment (start 177.375 61) (end 178.75 59.625) (width 0.2) (layer "F.Cu") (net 14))
 (segment (start 121.976 78.851) (end 121.25 78.125) (width 0.2) (layer "F.Cu") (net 13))
 (segment (start 164.774 78.851) (end 121.976 78.851) (width 0.2) (layer "F.Cu") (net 13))
 (segment (start 182.25 61.375) (end 164.774 78.851) (width 0.2) (layer "F.Cu") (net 13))
 (segment (start 128.625 79.875) (end 124.75 79.875) (width 0.2) (layer "F.Cu") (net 12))
 (segment (start 129 79.5) (end 128.625 79.875) (width 0.2) (layer "F.Cu") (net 12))
 (segment (start 130.626 78.125) (end 130.5 78.251) (width 0.2) (layer "F.Cu") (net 12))
 (segment (start 140.75 78.125) (end 130.626 78.125) (width 0.2) (layer "F.Cu") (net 12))
 (via (at 130.5 78.251) (size 0.6) (drill 0.3) (layers "F.Cu" "B.Cu") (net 12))
 (via (at 129 79.5) (size 0.6) (drill 0.3) (layers "F.Cu" "B.Cu") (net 12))
 (segment (start 130.249 78.251) (end 129 79.5) (width 0.2) (layer "B.Cu") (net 12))
 (segment (start 130.5 78.251) (end 130.249 78.251) (width 0.2) (layer "B.Cu") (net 12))
 (segment (start 119.19 48.96) (end 110.531142 48.96) (width 0.2) (layer "F.Cu") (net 10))
 (segment (start 110.531142 48.96) (end 108.455 51.036142) (width 0.2) (layer "F.Cu") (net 10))
 (segment (start 119.19 65.19) (end 111.5 57.5) (width 0.2) (layer "F.Cu") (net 9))
 (segment (start 119.19 67.96) (end 119.19 65.19) (width 0.2) (layer "F.Cu") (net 9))
 (via (at 111.5 57.5) (size 0.6) (drill 0.3) (layers "F.Cu" "B.Cu") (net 9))
 (segment (start 111.5 57.5) (end 107.62 53.62) (width 0.2) (layer "B.Cu") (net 9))
 (segment (start 107.62 53.62) (end 107.62 53.576142) (width 0.2) (layer "B.Cu") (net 9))
 (segment (start 112.519042 58.656142) (end 107.62 58.656142) (width 0.2) (layer "B.Cu") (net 20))
 (segment (start 122.215184 48.96) (end 112.519042 58.656142) (width 0.2) (layer "B.Cu") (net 20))
 (segment (start 138.36 48.96) (end 122.215184 48.96) (width 0.2) (layer "B.Cu") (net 20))
 (segment (start 111.5 61) (end 111.5 59.161142) (width 0.2) (layer "F.Cu") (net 15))
 (segment (start 111.5 59.161142) (end 108.455 56.116142) (width 0.2) (layer "F.Cu") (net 15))
 (via (at 111.5 61) (size 0.6) (drill 0.3) (layers "F.Cu" "B.Cu") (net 15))
 (segment (start 134.96 67.96) (end 129 62) (width 0.2) (layer "B.Cu") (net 15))
 (segment (start 112.5 62) (end 111.5 61) (width 0.2) (layer "B.Cu") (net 15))
 (segment (start 129 62) (end 112.5 62) (width 0.2) (layer "B.Cu") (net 15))
 (segment (start 138.29 67.96) (end 134.96 67.96) (width 0.2) (layer "B.Cu") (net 15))
 (segment (start 106.1 47.5) (end 105 47.5) (width 0.2) (layer "F.Cu") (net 5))
 (segment (start 157.53 48.96) (end 152.04 48.96) (width 0.2) (layer "F.Cu") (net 5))
 (segment (start 152.04 48.96) (end 152 49) (width 0.2) (layer "F.Cu") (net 5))
 (segment (start 105 47.5) (end 104 48.5) (width 0.2) (layer "F.Cu") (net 5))
 (via (at 106.1 47.5) (size 0.6) (drill 0.3) (layers "F.Cu" "B.Cu") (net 5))
 (via (at 152 49) (size 0.6) (drill 0.3) (layers "F.Cu" "B.Cu") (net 5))
 (via (at 104 48.5) (size 0.6) (drill 0.3) (layers "F.Cu" "B.Cu") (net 5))
 (segment (start 152 49) (end 140.381314 49) (width 0.2) (layer "B.Cu") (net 5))
 (segment (start 138.940314 47.559) (end 137.779686 47.559) (width 0.2) (layer "B.Cu") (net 5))
 (segment (start 106.566858 47.433142) (end 106.5 47.5) (width 0.2) (layer "B.Cu") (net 5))
 (segment (start 124.959686 47.821) (end 124.571828 47.433142) (width 0.2) (layer "B.Cu") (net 5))
 (segment (start 140.381314 49) (end 138.940314 47.559) (width 0.2) (layer "B.Cu") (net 5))
 (segment (start 106.5 47.5) (end 106.1 47.5) (width 0.2) (layer "B.Cu") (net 5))
 (segment (start 103.996142 48.496142) (end 92.38 48.496142) (width 0.2) (layer "B.Cu") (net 5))
 (segment (start 124.571828 47.433142) (end 106.566858 47.433142) (width 0.2) (layer "B.Cu") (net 5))
 (segment (start 137.779686 47.559) (end 137.517686 47.821) (width 0.2) (layer "B.Cu") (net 5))
 (segment (start 137.517686 47.821) (end 124.959686 47.821) (width 0.2) (layer "B.Cu") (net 5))
 (segment (start 104 48.5) (end 103.996142 48.496142) (width 0.2) (layer "B.Cu") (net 5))
 (segment (start 103.5 46.499452) (end 92.38 57.619452) (width 0.2) (layer "F.Cu") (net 19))
 (segment (start 103.5 43.5) (end 103.5 46.499452) (width 0.2) (layer "F.Cu") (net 19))
 (segment (start 92.38 57.619452) (end 92.38 58.656142) (width 0.2) (layer "F.Cu") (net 19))
 (via (at 103.5 43.5) (size 0.6) (drill 0.3) (layers "F.Cu" "B.Cu") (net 19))
 (segment (start 104.646858 42.353142) (end 103.5 43.5) (width 0.2) (layer "B.Cu") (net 19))
 (segment (start 170.083142 42.353142) (end 104.646858 42.353142) (width 0.2) (layer "B.Cu") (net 19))
 (segment (start 176.69 48.96) (end 170.083142 42.353142) (width 0.2) (layer "B.Cu") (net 19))
 (segment (start 116.899 81.399) (end 176.931 81.399) (width 0.2) (layer "F.Cu") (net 6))
 (segment (start 105.5 69.660108) (end 115.399 79.559108) (width 0.2) (layer "F.Cu") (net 6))
 (segment (start 115.399 79.899) (end 116.899 81.399) (width 0.2) (layer "F.Cu") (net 6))
 (segment (start 176.931 81.399) (end 189.1 69.23) (width 0.2) (layer "F.Cu") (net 6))
 (segment (start 105.5 53.5) (end 105.5 69.660108) (width 0.2) (layer "F.Cu") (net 6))
 (segment (start 115.399 79.559108) (end 115.399 79.899) (width 0.2) (layer "F.Cu") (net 6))
 (via (at 105.5 53.5) (size 0.6) (drill 0.3) (layers "F.Cu" "B.Cu") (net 6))
 (segment (start 105.5 45.536142) (end 107.62 43.416142) (width 0.2) (layer "B.Cu") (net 6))
 (segment (start 105.5 53.5) (end 105.5 45.536142) (width 0.2) (layer "B.Cu") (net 6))
 (segment (start 89.226 45.492512) (end 91.30237 43.416142) (width 0.2) (layer "F.Cu") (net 16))
 (segment (start 89.226 69.726) (end 89.226 45.492512) (width 0.2) (layer "F.Cu") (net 16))
 (segment (start 91.30237 43.416142) (end 92.38 43.416142) (width 0.2) (layer "F.Cu") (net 16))
 (segment (start 92.5 73) (end 89.226 69.726) (width 0.2) (layer "F.Cu") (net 16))
 (segment (start 188.91 74.5) (end 186 74.5) (width 0.2) (layer "F.Cu") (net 8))
 (segment (start 90.028 54.850512) (end 90.028 59.457768) (width 0.2) (layer "F.Cu") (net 8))
 (segment (start 92.070232 61.5) (end 92.5 61.5) (width 0.2) (layer "F.Cu") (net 8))
 (segment (start 91.30237 53.576142) (end 90.028 54.850512) (width 0.2) (layer "F.Cu") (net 8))
 (segment (start 92.38 53.576142) (end 91.30237 53.576142) (width 0.2) (layer "F.Cu") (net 8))
 (segment (start 189.1 74.31) (end 188.91 74.5) (width 0.2) (layer "F.Cu") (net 8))
 (segment (start 90.028 59.457768) (end 92.070232 61.5) (width 0.2) (layer "F.Cu") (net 8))
 (via (at 186 74.5) (size 0.6) (drill 0.3) (layers "F.Cu" "B.Cu") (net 8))
 (via (at 92.5 61.5) (size 0.6) (drill 0.3) (layers "F.Cu" "B.Cu") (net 8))
 (segment (start 186 74.5) (end 185.025353 74.5) (width 0.2) (layer "B.Cu") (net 8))
 (segment (start 178.126353 81.399) (end 113.399 81.399) (width 0.2) (layer "B.Cu") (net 8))
 (segment (start 92.557 61.443) (end 92.5 61.5) (width 0.2) (layer "B.Cu") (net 8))
 (segment (start 93.443 61.443) (end 92.557 61.443) (width 0.2) (layer "B.Cu") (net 8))
 (segment (start 113.399 81.399) (end 93.443 61.443) (width 0.2) (layer "B.Cu") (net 8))
 (segment (start 185.025353 74.5) (end 178.126353 81.399) (width 0.2) (layer "B.Cu") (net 8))
 (segment (start 184.77 71.77) (end 173 60) (width 0.2) (layer "B.Cu") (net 7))
 (segment (start 173 60) (end 96.263858 60) (width 0.2) (layer "B.Cu") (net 7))
 (segment (start 189.1 71.77) (end 184.77 71.77) (width 0.2) (layer "B.Cu") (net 7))
 (segment (start 96.263858 60) (end 92.38 56.116142) (width 0.2) (layer "B.Cu") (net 7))
 (segment (start 89.627 65.127) (end 89.627 47.631512) (width 0.2) (layer "F.Cu") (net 17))
 (segment (start 89.627 47.631512) (end 91.30237 45.956142) (width 0.2) (layer "F.Cu") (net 17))
 (segment (start 91.30237 45.956142) (end 92.38 45.956142) (width 0.2) (layer "F.Cu") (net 17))
 (segment (start 92.5 68) (end 89.627 65.127) (width 0.2) (layer "F.Cu") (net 17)))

